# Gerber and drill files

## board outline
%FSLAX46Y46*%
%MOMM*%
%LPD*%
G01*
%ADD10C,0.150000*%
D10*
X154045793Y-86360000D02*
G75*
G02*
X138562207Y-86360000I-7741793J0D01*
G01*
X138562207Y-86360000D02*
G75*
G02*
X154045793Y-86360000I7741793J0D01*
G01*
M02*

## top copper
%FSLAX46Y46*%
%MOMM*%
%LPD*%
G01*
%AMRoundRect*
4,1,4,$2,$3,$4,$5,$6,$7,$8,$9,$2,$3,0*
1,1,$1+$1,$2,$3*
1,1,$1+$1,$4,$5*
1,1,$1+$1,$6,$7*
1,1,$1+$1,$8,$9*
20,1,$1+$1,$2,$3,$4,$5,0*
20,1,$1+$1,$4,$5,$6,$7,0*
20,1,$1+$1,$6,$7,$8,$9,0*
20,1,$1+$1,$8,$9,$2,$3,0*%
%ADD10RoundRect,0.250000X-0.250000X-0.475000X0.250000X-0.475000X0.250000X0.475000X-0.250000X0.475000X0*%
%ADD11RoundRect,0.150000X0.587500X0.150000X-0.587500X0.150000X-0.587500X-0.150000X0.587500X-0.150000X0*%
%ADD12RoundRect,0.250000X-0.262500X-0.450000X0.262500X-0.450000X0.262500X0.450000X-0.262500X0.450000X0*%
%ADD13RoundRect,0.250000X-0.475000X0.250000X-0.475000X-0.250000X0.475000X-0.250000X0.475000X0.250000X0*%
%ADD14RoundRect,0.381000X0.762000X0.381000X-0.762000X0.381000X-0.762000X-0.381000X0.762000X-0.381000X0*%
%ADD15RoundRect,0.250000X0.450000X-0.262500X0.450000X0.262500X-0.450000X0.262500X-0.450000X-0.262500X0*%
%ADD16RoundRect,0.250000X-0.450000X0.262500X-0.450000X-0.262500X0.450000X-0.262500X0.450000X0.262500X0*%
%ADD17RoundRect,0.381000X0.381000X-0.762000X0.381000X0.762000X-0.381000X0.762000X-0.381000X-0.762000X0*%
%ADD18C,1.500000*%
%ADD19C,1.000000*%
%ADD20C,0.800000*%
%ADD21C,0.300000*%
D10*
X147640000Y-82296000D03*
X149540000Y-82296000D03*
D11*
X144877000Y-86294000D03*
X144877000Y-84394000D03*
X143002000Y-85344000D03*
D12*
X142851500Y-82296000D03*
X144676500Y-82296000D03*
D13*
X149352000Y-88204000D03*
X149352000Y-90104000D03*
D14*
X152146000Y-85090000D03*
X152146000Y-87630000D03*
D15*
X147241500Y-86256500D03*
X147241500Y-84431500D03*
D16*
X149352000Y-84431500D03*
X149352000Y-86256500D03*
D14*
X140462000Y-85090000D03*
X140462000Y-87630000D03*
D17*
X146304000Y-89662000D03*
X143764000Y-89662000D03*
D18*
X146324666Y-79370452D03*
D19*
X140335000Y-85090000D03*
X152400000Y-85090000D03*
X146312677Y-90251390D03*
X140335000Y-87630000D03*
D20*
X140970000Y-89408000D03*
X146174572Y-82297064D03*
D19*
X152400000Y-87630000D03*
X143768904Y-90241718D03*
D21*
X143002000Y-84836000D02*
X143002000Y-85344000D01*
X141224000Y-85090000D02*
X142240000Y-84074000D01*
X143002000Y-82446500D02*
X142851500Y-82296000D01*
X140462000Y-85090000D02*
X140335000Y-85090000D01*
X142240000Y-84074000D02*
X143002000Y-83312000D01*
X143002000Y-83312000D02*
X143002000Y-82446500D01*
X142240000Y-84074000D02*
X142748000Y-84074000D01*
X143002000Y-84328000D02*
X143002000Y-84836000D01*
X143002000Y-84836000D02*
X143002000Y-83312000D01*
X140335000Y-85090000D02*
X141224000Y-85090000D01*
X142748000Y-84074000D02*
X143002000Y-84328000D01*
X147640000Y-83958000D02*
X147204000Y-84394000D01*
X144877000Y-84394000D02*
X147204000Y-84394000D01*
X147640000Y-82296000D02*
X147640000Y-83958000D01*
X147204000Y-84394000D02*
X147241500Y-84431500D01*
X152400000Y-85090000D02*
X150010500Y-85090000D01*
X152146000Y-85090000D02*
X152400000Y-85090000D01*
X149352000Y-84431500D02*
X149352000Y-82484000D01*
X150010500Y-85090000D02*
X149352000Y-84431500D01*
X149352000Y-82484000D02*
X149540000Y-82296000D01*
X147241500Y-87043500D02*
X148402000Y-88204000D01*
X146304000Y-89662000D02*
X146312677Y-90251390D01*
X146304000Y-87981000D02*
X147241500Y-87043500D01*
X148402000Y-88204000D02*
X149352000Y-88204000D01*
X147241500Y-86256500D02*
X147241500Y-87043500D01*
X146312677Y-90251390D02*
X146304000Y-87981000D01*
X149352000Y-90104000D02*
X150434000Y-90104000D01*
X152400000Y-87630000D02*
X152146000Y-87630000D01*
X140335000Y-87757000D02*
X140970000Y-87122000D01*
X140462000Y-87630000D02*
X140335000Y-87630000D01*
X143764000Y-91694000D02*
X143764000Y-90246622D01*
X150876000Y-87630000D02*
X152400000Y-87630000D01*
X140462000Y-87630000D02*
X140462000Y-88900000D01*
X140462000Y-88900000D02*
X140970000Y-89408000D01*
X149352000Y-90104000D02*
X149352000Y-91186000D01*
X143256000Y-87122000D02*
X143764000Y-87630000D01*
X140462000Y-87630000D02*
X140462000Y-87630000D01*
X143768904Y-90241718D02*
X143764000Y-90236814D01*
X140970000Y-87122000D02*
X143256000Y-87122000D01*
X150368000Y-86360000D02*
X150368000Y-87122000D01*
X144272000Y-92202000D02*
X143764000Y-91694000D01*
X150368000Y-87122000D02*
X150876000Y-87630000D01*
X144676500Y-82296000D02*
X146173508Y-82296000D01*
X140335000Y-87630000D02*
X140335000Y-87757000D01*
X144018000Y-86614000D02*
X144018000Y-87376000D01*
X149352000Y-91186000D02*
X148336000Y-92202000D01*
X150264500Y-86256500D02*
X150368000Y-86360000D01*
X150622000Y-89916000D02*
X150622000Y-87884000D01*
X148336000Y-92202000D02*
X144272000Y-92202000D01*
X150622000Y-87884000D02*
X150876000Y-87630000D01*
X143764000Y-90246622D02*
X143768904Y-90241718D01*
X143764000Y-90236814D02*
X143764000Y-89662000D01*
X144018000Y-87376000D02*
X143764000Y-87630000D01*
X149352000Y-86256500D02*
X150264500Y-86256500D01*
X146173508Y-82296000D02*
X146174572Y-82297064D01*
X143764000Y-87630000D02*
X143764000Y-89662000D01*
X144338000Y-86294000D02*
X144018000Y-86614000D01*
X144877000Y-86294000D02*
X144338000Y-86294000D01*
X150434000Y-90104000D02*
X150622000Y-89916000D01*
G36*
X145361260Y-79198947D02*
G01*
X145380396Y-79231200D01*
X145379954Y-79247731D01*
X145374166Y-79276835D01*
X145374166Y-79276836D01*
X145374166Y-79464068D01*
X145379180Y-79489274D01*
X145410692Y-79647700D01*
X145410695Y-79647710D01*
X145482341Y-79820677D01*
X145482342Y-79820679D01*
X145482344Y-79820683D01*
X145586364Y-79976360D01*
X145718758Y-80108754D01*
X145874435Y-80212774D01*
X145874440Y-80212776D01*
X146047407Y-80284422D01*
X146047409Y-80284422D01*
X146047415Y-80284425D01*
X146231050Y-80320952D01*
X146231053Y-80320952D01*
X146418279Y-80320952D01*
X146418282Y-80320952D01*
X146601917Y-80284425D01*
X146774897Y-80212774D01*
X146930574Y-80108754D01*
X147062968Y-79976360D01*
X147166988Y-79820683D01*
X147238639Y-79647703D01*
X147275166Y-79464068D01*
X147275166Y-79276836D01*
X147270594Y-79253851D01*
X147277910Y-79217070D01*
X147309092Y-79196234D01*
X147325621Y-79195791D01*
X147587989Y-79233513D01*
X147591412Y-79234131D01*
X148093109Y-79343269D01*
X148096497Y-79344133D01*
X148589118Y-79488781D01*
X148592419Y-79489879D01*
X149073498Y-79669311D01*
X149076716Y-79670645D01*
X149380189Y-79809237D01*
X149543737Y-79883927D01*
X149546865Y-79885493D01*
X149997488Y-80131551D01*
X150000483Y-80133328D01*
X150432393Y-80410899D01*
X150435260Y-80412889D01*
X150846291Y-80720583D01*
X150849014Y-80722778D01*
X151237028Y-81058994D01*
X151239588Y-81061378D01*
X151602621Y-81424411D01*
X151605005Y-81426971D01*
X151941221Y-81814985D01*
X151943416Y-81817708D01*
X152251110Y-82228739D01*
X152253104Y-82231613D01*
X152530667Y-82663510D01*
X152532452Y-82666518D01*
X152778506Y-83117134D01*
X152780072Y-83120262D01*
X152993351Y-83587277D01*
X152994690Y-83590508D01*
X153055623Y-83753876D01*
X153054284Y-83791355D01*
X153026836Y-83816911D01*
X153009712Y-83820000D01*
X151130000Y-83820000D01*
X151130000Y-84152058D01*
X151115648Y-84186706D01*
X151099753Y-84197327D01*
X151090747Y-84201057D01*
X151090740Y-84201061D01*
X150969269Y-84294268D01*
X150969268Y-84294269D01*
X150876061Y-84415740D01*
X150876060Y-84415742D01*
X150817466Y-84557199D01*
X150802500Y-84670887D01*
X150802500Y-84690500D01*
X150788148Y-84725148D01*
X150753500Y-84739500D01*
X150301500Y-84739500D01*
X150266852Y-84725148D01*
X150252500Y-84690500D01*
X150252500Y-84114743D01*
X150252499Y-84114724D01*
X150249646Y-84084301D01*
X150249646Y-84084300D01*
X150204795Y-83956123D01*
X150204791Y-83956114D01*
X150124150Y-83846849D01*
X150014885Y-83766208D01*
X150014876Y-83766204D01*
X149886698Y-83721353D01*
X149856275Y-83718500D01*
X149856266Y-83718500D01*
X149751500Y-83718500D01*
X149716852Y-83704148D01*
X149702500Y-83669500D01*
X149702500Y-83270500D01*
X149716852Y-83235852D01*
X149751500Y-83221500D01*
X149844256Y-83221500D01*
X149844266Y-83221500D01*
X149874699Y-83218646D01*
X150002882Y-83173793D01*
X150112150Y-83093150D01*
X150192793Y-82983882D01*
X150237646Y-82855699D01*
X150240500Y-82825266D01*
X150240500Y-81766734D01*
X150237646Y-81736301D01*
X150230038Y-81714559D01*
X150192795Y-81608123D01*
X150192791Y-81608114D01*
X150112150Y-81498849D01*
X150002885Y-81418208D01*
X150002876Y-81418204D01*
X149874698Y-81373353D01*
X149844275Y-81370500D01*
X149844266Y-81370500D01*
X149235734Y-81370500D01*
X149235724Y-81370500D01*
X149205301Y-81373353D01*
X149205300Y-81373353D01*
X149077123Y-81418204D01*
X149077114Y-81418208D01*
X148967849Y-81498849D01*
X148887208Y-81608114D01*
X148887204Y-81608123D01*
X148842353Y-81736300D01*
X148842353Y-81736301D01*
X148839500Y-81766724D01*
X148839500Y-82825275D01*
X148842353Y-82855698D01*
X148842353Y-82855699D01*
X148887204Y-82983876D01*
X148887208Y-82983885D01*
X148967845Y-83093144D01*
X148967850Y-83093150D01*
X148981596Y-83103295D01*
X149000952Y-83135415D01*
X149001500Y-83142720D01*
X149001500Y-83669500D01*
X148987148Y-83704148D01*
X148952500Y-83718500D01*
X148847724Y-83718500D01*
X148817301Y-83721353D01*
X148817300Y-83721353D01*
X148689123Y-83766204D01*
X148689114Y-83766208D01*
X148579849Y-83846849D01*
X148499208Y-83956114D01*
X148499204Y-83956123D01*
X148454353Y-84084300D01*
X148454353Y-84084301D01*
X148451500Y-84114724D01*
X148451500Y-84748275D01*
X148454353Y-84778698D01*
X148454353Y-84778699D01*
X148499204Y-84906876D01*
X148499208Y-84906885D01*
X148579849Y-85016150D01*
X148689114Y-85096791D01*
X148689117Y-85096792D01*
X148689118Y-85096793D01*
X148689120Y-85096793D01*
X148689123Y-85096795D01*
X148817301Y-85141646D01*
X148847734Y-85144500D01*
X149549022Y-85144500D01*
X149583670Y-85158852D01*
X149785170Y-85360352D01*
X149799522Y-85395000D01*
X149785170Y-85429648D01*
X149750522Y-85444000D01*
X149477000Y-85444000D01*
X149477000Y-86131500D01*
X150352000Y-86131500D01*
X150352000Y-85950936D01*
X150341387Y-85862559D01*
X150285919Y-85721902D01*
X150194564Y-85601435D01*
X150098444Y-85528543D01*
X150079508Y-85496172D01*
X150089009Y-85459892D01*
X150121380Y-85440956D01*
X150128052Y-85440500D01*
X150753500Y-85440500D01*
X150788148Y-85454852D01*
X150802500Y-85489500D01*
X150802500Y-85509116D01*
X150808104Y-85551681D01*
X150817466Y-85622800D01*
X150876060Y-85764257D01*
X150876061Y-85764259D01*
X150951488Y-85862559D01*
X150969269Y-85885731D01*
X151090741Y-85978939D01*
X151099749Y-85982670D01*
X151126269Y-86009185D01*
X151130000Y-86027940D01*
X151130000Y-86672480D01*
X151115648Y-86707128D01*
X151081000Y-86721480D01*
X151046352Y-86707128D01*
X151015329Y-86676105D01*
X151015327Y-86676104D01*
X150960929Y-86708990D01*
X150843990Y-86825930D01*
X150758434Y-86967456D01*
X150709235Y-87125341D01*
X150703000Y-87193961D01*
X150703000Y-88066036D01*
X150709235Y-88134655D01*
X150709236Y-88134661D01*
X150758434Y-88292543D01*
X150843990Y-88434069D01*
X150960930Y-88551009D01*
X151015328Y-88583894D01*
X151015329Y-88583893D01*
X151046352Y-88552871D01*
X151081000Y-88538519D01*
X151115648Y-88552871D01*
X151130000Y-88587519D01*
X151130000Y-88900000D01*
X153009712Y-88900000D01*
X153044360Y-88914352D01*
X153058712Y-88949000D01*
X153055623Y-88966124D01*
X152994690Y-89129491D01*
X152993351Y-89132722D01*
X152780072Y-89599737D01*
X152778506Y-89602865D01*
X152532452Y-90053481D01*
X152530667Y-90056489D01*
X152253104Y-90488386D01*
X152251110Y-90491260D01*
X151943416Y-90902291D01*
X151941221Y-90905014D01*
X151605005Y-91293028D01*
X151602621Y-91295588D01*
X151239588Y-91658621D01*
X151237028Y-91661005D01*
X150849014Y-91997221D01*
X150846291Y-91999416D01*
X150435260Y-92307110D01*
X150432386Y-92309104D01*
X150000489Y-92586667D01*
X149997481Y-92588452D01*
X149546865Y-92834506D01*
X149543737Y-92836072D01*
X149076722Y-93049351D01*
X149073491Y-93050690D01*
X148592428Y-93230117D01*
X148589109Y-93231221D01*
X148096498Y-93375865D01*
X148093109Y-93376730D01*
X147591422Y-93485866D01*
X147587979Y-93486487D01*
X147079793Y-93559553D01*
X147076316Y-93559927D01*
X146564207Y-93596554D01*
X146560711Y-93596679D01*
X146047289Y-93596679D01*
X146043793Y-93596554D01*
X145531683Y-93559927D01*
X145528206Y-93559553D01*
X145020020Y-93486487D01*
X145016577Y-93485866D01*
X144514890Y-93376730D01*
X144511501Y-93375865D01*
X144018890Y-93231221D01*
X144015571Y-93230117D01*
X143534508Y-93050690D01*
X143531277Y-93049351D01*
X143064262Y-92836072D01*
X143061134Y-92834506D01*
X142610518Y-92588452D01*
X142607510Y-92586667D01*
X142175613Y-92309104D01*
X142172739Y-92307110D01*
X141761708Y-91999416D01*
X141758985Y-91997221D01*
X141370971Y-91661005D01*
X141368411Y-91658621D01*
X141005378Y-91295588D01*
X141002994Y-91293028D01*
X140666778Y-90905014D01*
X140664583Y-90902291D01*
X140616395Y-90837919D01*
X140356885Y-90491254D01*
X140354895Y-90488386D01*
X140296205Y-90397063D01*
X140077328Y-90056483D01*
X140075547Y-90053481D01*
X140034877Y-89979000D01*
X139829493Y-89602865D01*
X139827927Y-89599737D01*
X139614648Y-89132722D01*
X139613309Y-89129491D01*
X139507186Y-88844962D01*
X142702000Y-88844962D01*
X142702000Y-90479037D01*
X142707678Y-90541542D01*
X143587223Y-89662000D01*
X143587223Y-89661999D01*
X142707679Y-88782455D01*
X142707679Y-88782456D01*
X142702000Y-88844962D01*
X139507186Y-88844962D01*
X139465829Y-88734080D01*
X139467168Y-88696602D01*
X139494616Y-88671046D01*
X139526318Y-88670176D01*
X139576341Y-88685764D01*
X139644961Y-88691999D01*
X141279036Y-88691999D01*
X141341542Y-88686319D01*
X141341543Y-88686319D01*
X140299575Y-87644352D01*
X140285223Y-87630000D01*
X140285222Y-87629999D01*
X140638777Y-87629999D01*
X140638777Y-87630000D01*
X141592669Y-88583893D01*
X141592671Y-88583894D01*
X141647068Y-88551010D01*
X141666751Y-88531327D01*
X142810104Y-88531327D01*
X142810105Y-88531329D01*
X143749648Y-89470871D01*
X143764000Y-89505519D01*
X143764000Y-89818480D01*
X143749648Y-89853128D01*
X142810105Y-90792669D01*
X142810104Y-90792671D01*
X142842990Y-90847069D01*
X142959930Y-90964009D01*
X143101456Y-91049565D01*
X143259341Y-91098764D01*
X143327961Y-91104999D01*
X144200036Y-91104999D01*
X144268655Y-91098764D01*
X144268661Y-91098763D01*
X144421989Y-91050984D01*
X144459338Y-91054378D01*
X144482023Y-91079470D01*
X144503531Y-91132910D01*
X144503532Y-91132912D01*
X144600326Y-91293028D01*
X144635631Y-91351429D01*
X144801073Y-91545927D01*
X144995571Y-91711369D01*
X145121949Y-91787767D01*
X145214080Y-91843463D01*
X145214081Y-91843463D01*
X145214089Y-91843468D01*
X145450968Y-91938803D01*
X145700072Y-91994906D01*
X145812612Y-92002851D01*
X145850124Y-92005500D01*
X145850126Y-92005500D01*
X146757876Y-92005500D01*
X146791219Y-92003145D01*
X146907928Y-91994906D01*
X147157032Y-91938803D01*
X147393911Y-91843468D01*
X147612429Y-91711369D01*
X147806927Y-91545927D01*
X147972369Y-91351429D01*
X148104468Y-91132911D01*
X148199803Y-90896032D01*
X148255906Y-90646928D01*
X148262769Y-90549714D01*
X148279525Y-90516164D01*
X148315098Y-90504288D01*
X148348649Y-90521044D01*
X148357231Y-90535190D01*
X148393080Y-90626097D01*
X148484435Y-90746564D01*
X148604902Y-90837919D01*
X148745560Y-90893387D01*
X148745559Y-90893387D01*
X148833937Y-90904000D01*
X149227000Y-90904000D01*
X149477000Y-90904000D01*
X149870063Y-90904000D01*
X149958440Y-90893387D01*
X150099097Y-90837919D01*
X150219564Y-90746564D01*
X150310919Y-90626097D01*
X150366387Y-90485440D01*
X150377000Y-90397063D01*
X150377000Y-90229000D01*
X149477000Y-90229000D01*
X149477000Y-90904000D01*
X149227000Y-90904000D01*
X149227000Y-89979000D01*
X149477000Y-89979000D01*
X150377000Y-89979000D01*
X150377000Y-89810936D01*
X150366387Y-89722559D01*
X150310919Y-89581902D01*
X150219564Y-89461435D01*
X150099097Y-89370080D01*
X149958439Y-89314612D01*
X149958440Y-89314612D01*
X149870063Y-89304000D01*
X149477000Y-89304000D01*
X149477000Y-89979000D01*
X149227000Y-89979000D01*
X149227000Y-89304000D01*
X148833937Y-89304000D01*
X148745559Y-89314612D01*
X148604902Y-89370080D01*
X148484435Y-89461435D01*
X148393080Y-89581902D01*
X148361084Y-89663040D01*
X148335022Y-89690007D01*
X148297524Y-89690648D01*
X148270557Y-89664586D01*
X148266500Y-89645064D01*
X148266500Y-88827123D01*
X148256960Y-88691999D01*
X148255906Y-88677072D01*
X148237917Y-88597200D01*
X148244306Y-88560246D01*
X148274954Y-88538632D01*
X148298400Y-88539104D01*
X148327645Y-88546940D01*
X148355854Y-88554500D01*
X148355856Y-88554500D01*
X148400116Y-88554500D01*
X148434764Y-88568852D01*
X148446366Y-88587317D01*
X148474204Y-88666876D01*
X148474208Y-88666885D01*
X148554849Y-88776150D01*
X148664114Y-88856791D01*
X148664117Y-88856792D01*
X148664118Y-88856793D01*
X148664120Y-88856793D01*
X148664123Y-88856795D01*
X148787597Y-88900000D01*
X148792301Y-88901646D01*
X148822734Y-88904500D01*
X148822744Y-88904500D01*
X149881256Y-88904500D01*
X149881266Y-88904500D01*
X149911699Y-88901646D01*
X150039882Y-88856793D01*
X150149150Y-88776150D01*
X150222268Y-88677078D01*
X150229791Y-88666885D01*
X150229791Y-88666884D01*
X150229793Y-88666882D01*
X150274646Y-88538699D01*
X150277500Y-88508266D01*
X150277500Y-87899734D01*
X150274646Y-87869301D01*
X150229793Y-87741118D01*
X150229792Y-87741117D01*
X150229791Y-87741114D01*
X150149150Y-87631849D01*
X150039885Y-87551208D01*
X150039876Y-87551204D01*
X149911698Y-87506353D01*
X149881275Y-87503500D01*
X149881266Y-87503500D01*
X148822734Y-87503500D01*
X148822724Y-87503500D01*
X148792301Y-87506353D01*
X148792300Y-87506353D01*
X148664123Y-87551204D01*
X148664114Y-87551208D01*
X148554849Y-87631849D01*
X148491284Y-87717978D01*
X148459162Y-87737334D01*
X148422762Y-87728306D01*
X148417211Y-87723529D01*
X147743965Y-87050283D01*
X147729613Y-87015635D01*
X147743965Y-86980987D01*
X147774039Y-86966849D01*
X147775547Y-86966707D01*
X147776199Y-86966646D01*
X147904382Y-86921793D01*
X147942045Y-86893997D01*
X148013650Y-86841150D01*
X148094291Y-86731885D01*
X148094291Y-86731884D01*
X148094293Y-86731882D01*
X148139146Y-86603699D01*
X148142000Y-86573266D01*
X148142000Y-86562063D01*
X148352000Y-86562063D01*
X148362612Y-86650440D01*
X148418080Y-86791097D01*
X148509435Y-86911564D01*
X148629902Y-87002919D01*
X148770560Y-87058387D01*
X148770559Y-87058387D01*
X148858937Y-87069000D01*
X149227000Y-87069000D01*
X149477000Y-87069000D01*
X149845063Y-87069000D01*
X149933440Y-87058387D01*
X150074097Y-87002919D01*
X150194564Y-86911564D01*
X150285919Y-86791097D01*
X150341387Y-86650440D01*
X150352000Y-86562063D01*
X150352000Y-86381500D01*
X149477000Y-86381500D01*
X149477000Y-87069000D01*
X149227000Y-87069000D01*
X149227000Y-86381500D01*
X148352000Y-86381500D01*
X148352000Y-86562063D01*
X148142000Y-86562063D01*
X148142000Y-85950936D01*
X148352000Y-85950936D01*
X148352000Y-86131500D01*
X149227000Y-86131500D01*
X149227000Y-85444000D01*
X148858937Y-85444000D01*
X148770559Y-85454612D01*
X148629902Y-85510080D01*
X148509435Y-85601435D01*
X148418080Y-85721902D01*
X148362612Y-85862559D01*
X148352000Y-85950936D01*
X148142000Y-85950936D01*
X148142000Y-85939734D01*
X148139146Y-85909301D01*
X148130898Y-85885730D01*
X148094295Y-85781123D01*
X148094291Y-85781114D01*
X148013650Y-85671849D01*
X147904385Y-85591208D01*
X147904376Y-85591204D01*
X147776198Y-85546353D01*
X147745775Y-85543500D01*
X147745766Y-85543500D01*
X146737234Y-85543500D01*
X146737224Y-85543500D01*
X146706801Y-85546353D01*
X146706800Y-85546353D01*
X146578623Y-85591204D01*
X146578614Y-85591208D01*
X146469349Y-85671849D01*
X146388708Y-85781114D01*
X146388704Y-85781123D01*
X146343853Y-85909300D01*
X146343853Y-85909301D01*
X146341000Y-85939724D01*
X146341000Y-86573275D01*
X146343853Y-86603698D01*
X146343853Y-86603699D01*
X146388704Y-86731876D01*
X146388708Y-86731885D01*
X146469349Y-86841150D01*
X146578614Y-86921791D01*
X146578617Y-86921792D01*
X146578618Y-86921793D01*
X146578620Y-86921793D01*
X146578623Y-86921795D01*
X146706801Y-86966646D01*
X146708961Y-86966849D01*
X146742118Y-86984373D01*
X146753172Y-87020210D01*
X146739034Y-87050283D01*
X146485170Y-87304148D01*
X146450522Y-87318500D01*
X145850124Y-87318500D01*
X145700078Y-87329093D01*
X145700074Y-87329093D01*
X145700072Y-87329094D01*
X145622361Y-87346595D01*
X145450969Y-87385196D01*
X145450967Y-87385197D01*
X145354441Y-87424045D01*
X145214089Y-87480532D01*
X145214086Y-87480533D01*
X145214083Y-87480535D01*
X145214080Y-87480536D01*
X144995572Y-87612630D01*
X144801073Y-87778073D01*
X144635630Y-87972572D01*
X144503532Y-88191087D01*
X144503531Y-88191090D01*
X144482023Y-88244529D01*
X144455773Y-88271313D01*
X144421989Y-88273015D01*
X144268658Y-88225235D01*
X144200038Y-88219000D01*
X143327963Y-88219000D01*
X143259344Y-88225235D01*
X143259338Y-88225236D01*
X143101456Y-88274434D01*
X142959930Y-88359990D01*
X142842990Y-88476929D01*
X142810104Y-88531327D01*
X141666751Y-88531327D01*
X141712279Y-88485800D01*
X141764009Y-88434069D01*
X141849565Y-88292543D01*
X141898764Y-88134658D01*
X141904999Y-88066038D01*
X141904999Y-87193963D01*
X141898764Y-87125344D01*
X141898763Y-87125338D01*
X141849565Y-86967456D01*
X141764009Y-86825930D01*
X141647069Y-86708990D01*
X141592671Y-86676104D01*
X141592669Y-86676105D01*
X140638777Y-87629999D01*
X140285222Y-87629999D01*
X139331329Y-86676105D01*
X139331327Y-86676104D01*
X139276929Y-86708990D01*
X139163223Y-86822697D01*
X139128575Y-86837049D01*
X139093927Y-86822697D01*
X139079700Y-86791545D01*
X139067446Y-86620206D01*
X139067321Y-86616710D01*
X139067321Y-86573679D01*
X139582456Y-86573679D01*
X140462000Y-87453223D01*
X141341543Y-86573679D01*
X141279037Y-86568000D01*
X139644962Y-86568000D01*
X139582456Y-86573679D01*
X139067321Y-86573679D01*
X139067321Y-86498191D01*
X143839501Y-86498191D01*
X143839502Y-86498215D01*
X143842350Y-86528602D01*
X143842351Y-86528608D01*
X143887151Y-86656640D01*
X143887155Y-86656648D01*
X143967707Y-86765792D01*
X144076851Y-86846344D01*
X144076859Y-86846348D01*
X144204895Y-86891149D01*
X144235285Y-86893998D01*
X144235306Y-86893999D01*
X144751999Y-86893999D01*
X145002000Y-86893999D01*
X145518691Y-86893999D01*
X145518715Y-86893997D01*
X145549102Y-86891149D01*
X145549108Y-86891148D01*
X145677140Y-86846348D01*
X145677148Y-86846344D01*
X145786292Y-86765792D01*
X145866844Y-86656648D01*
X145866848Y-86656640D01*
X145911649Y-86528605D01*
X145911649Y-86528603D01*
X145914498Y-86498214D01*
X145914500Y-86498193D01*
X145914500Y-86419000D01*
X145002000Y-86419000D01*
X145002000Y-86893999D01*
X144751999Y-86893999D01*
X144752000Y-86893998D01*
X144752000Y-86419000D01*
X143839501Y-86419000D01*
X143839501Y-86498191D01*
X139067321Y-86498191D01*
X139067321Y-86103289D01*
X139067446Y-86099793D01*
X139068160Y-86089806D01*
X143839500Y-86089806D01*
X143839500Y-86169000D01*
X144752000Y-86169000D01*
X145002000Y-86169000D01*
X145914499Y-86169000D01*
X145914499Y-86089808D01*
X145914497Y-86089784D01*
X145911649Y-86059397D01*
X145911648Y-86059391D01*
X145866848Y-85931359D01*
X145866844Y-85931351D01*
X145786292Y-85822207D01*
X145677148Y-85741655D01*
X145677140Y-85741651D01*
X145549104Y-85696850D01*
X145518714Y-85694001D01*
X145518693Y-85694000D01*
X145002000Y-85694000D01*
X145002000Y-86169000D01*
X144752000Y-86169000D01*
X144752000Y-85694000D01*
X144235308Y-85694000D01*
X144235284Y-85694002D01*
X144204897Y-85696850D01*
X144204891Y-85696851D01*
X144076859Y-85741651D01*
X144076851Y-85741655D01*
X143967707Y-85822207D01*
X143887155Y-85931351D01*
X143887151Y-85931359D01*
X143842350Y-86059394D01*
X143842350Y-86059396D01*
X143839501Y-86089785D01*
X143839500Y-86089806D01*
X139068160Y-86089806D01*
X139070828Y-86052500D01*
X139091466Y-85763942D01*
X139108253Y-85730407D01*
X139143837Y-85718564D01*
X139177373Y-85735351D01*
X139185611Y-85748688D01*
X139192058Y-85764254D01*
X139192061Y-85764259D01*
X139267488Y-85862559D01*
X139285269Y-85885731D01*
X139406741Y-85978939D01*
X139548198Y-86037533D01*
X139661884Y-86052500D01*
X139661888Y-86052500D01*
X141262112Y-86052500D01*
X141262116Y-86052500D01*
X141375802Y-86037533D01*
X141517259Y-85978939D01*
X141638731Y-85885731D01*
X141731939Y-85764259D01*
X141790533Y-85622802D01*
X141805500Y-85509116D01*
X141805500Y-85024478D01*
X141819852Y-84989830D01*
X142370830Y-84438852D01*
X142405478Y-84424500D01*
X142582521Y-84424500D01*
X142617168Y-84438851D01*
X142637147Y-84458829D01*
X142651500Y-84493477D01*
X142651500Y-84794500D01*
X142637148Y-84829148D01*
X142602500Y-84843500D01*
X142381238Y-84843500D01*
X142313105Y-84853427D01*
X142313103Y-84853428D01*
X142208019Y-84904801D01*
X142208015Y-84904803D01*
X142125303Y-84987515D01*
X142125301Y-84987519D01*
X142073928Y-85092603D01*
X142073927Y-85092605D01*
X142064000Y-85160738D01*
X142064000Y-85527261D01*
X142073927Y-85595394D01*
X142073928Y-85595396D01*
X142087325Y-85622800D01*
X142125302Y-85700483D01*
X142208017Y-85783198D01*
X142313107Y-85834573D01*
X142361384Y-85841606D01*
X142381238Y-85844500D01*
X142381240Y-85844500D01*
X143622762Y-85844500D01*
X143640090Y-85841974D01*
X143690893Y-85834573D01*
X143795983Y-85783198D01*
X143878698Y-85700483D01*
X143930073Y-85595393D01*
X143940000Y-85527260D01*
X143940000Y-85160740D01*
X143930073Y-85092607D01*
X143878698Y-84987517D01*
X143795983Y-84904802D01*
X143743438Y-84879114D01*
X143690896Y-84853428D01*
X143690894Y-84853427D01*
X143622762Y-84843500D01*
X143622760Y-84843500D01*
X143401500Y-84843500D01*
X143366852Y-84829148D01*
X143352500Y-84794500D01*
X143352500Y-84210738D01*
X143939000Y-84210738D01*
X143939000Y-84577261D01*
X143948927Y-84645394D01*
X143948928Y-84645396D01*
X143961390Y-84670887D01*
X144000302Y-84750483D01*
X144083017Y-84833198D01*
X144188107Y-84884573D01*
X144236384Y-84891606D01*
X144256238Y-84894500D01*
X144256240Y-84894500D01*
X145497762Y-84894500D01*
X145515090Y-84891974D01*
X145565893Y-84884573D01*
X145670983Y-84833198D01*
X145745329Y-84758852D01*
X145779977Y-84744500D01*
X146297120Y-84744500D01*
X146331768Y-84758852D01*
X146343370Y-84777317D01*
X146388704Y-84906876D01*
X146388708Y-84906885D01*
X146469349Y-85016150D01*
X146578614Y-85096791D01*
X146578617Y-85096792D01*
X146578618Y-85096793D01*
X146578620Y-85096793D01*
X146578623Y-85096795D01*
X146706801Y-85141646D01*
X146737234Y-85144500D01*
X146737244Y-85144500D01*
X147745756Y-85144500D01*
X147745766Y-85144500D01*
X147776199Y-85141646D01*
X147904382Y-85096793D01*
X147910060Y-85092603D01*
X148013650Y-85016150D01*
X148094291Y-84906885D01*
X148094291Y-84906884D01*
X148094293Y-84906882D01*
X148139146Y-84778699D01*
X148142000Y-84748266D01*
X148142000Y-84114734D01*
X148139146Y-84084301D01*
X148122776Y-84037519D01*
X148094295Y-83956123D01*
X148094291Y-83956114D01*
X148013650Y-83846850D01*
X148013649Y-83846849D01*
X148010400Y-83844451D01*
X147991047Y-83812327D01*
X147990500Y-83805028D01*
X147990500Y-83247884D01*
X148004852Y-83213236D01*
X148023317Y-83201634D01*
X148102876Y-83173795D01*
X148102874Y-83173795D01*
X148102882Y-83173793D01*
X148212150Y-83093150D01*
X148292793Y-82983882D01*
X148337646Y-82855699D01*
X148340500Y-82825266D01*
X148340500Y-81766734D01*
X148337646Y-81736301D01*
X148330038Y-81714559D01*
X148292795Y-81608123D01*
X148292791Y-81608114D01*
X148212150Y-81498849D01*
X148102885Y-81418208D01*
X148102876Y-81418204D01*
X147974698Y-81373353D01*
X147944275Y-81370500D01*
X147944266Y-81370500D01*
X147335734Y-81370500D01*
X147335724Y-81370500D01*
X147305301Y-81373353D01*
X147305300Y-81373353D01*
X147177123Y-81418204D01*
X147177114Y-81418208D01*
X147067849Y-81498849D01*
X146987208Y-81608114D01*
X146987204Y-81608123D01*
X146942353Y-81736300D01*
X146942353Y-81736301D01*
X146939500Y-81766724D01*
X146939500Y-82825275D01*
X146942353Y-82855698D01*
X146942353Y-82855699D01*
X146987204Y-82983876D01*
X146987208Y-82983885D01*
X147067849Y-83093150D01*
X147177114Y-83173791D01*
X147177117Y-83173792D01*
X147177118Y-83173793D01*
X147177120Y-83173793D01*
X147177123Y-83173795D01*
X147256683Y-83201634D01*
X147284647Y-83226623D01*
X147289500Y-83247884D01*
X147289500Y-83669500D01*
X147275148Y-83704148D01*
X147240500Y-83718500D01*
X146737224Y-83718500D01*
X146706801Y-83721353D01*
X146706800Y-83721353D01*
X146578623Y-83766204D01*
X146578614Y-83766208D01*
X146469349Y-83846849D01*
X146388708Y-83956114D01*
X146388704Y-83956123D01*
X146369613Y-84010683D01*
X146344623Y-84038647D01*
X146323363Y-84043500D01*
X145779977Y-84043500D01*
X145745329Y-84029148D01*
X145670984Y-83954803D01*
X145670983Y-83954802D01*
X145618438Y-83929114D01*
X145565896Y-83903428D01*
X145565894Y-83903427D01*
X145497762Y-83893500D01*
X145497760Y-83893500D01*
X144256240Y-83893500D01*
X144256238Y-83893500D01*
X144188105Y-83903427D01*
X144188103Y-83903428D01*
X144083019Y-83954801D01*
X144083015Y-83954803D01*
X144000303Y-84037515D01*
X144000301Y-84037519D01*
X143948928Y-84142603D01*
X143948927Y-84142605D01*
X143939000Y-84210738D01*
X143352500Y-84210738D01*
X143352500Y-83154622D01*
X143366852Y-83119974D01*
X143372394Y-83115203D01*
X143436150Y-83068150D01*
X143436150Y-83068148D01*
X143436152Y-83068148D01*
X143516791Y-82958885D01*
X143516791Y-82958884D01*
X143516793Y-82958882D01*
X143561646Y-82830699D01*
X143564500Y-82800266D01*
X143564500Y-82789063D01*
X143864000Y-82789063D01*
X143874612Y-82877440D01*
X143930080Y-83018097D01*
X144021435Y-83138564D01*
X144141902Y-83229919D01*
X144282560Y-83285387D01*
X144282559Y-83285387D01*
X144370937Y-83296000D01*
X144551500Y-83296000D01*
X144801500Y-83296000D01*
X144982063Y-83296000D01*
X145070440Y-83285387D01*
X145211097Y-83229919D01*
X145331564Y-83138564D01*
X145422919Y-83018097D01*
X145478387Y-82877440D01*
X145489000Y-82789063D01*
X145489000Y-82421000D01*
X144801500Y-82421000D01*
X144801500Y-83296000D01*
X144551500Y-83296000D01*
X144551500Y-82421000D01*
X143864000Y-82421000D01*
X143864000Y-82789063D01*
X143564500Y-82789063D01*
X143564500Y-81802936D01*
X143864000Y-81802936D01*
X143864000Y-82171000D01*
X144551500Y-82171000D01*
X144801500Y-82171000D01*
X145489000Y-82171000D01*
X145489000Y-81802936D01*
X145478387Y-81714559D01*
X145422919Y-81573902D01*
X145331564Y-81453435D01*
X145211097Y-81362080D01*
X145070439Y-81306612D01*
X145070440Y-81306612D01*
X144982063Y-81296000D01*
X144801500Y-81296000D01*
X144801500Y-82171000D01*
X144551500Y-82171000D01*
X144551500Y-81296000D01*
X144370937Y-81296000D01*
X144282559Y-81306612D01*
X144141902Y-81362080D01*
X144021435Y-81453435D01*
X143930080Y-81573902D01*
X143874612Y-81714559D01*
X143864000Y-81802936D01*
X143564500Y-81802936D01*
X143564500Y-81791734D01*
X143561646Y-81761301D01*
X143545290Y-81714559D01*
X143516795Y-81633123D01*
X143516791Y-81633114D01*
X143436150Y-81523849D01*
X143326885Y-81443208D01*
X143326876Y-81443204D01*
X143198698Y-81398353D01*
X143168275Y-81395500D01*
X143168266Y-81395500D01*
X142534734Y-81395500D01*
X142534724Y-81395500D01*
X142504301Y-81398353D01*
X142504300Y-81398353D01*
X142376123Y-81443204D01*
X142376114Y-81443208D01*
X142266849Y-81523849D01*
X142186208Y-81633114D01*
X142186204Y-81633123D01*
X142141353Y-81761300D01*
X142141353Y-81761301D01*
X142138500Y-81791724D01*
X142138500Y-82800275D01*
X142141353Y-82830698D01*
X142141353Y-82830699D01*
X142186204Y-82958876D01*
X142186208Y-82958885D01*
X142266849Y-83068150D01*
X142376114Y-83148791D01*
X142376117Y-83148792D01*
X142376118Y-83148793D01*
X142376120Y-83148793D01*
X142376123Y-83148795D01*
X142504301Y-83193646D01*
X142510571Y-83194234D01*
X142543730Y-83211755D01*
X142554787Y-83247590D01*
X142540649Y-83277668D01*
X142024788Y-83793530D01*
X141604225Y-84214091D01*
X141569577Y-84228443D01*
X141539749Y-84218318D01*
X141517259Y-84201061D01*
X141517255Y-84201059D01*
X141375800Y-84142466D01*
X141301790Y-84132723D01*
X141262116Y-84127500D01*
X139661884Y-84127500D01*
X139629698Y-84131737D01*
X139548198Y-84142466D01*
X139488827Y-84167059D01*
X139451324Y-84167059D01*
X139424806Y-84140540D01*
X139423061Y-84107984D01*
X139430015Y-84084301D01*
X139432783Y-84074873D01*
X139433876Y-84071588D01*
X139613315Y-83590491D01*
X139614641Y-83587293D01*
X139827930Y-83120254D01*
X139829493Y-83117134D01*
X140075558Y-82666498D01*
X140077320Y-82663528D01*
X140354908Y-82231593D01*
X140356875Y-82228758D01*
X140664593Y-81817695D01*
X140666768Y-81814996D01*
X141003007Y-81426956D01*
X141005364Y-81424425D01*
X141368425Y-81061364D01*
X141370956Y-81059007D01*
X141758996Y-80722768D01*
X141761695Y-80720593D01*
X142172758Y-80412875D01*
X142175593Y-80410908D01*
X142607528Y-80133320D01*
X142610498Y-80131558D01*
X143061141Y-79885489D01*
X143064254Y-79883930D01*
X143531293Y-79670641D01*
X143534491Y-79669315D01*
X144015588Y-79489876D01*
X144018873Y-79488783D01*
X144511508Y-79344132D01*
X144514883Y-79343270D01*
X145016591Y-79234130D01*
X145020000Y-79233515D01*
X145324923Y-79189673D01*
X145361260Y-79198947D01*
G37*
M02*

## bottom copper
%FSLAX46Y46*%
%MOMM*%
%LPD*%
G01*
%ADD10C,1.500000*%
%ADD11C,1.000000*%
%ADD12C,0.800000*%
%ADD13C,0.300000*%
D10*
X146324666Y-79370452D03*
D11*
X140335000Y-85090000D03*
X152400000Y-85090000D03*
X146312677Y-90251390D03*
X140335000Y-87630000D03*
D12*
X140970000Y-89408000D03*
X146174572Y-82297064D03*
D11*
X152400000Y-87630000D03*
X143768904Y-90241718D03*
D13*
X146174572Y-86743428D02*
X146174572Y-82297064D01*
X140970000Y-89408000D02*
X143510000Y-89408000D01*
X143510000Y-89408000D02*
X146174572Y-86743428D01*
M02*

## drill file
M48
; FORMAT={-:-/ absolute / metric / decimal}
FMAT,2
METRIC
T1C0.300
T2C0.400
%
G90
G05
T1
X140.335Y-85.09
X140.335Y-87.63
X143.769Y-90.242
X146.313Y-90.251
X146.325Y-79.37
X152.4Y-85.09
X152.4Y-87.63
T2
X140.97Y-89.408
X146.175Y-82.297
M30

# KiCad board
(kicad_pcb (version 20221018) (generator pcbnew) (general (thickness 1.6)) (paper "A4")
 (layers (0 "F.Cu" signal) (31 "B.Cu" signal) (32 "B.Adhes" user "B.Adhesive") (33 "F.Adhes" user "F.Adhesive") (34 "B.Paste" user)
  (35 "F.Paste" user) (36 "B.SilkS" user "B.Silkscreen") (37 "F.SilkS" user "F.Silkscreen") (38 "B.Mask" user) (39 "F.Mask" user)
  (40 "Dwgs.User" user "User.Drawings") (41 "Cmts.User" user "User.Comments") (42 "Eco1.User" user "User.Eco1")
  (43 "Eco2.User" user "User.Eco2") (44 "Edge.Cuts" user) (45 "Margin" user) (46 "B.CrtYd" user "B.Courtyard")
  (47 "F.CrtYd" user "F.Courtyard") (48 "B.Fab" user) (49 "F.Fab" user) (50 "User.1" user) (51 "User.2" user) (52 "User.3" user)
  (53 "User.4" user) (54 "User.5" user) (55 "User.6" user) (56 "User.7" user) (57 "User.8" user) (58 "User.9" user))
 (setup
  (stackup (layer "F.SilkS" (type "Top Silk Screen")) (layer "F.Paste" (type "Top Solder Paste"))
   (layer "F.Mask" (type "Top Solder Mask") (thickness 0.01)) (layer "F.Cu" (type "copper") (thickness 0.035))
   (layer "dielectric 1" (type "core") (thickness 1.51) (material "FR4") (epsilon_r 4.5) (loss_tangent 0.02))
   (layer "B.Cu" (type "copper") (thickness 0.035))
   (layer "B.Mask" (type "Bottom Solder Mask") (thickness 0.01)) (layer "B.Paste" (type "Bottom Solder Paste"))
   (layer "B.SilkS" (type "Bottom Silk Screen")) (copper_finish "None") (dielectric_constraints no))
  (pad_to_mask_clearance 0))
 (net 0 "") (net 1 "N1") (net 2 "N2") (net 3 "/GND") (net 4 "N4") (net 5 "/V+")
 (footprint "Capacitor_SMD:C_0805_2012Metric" (layer "F.Cu") (at 148.59 82.296)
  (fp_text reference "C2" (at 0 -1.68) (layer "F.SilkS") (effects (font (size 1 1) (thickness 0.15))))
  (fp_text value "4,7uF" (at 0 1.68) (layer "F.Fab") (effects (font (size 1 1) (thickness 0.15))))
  (pad "1" smd roundrect (at -0.95 0) (size 1 1.45) (layers "F.Cu" "F.Paste" "F.Mask") (roundrect_rratio 0.25) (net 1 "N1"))
  (pad "2" smd roundrect (at 0.95 0) (size 1 1.45) (layers "F.Cu" "F.Paste" "F.Mask") (roundrect_rratio 0.25) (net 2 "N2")))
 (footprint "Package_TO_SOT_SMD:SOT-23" (layer "F.Cu") (at 143.9395 85.344 180)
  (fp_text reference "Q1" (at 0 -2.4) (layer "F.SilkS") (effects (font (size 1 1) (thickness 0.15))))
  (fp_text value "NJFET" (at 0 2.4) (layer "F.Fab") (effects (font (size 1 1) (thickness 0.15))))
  (pad "1" smd roundrect (at -0.9375 -0.95 180) (size 1.475 0.6) (layers "F.Cu" "F.Paste" "F.Mask") (roundrect_rratio 0.25) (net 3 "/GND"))
  (pad "2" smd roundrect (at -0.9375 0.95 180) (size 1.475 0.6) (layers "F.Cu" "F.Paste" "F.Mask") (roundrect_rratio 0.25) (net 1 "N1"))
  (pad "3" smd roundrect (at 0.9375 0 180) (size 1.475 0.6) (layers "F.Cu" "F.Paste" "F.Mask") (roundrect_rratio 0.25) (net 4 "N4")))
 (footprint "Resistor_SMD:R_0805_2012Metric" (layer "F.Cu") (at 143.764 82.296)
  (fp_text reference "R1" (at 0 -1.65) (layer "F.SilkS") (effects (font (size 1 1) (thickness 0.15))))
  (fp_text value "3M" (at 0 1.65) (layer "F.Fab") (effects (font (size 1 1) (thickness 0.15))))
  (pad "1" smd roundrect (at -0.9125 0) (size 1.025 1.4) (layers "F.Cu" "F.Paste" "F.Mask") (roundrect_rratio 0.243902) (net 4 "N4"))
  (pad "2" smd roundrect (at 0.9125 0) (size 1.025 1.4) (layers "F.Cu" "F.Paste" "F.Mask") (roundrect_rratio 0.243902) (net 3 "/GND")))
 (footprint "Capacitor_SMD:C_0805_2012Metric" (layer "F.Cu") (at 149.352 89.154 -90)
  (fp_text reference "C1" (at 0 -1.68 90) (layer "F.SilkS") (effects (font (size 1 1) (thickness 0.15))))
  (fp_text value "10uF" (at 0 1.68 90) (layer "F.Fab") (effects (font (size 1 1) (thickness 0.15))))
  (pad "1" smd roundrect (at -0.95 0 270) (size 1 1.45) (layers "F.Cu" "F.Paste" "F.Mask") (roundrect_rratio 0.25) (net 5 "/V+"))
  (pad "2" smd roundrect (at 0.95 0 270) (size 1 1.45) (layers "F.Cu" "F.Paste" "F.Mask") (roundrect_rratio 0.25) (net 3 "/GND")))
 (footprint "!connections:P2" (layer "F.Cu") (at 152.146 85.09 180)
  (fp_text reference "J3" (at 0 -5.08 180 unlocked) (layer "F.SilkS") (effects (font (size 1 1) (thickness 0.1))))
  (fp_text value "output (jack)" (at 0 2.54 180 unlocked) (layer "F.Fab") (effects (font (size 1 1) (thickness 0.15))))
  (pad "1" smd roundrect (at 0 0 180) (size 2.286 1.524) (layers "F.Cu" "F.Paste" "F.Mask") (roundrect_rratio 0.25) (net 2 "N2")
   (thermal_bridge_angle 45))
  (pad "2" smd roundrect (at 0 -2.54 180) (size 2.286 1.524) (layers "F.Cu" "F.Paste" "F.Mask") (roundrect_rratio 0.25) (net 3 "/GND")
   (thermal_bridge_angle 45)))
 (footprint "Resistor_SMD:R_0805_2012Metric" (layer "F.Cu") (at 147.2415 85.344 90)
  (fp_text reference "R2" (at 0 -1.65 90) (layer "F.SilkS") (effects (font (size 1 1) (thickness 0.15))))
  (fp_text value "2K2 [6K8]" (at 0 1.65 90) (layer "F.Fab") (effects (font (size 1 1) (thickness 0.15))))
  (pad "1" smd roundrect (at -0.9125 0 90) (size 1.025 1.4) (layers "F.Cu" "F.Paste" "F.Mask") (roundrect_rratio 0.243902) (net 5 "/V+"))
  (pad "2" smd roundrect (at 0.9125 0 90) (size 1.025 1.4) (layers "F.Cu" "F.Paste" "F.Mask") (roundrect_rratio 0.243902) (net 1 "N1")))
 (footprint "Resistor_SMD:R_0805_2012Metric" (layer "F.Cu") (at 149.352 85.344 -90)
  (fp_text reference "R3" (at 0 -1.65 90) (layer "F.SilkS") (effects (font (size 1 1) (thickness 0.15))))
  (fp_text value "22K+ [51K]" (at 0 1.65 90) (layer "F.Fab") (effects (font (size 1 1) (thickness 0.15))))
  (pad "1" smd roundrect (at -0.9125 0 270) (size 1.025 1.4) (layers "F.Cu" "F.Paste" "F.Mask") (roundrect_rratio 0.243902) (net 2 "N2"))
  (pad "2" smd roundrect (at 0.9125 0 270) (size 1.025 1.4) (layers "F.Cu" "F.Paste" "F.Mask") (roundrect_rratio 0.243902) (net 3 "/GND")))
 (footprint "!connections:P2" (layer "F.Cu") (at 140.462 85.09 180)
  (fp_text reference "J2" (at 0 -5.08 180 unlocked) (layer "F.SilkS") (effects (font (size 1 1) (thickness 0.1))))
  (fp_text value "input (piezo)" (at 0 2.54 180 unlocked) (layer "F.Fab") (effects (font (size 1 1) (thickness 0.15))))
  (pad "1" smd roundrect (at 0 0 180) (size 2.286 1.524) (layers "F.Cu" "F.Paste" "F.Mask") (roundrect_rratio 0.25) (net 4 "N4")
   (thermal_bridge_angle 45))
  (pad "2" smd roundrect (at 0 -2.54 180) (size 2.286 1.524) (layers "F.Cu" "F.Paste" "F.Mask") (roundrect_rratio 0.25) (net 3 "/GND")
   (thermal_bridge_angle 45)))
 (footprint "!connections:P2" (layer "F.Cu") (at 146.304 89.662 90) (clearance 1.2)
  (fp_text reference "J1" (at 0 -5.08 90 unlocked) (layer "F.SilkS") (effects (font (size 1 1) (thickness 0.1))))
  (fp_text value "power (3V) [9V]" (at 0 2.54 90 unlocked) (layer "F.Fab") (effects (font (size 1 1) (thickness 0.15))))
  (pad "1" smd roundrect (at 0 0 90) (size 2.286 1.524) (layers "F.Cu" "F.Paste" "F.Mask") (roundrect_rratio 0.25) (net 5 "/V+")
   (thermal_bridge_angle 45))
  (pad "2" smd roundrect (at 0 -2.54 90) (size 2.286 1.524) (layers "F.Cu" "F.Paste" "F.Mask") (roundrect_rratio 0.25) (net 3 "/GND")
   (thermal_bridge_angle 45)))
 (gr_circle (center 146.304 86.36) (end 151.384 80.518) (stroke (width 0.15) (type default)) (fill none) (layer "Edge.Cuts"))
 (via (at 146.324666 79.370452) (size 1.5) (drill 0.3) (layers "F.Cu" "B.Cu") (free) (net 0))
 (segment (start 143.002 84.836) (end 143.002 85.344) (width 0.3) (layer "F.Cu") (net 4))
 (segment (start 141.224 85.09) (end 142.24 84.074) (width 0.3) (layer "F.Cu") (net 4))
 (segment (start 143.002 82.4465) (end 142.8515 82.296) (width 0.3) (layer "F.Cu") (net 4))
 (segment (start 140.462 85.09) (end 140.335 85.09) (width 0.3) (layer "F.Cu") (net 4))
 (segment (start 142.24 84.074) (end 143.002 83.312) (width 0.3) (layer "F.Cu") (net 4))
 (segment (start 143.002 83.312) (end 143.002 82.4465) (width 0.3) (layer "F.Cu") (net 4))
 (segment (start 142.24 84.074) (end 142.748 84.074) (width 0.3) (layer "F.Cu") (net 4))
 (segment (start 143.002 84.328) (end 143.002 84.836) (width 0.3) (layer "F.Cu") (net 4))
 (segment (start 143.002 84.836) (end 143.002 83.312) (width 0.3) (layer "F.Cu") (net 4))
 (segment (start 140.335 85.09) (end 141.224 85.09) (width 0.3) (layer "F.Cu") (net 4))
 (segment (start 142.748 84.074) (end 143.002 84.328) (width 0.3) (layer "F.Cu") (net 4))
 (via (at 140.335 85.09) (size 1) (drill 0.3) (layers "F.Cu" "B.Cu") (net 4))
 (segment (start 147.64 83.958) (end 147.204 84.394) (width 0.3) (layer "F.Cu") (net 1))
 (segment (start 144.877 84.394) (end 147.204 84.394) (width 0.3) (layer "F.Cu") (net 1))
 (segment (start 147.64 82.296) (end 147.64 83.958) (width 0.3) (layer "F.Cu") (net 1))
 (segment (start 147.204 84.394) (end 147.2415 84.4315) (width 0.3) (layer "F.Cu") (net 1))
 (segment (start 152.4 85.09) (end 150.0105 85.09) (width 0.3) (layer "F.Cu") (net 2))
 (segment (start 152.146 85.09) (end 152.4 85.09) (width 0.3) (layer "F.Cu") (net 2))
 (segment (start 149.352 84.4315) (end 149.352 82.484) (width 0.3) (layer "F.Cu") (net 2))
 (segment (start 150.0105 85.09) (end 149.352 84.4315) (width 0.3) (layer "F.Cu") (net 2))
 (segment (start 149.352 82.484) (end 149.54 82.296) (width 0.3) (layer "F.Cu") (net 2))
 (via (at 152.4 85.09) (size 1) (drill 0.3) (layers "F.Cu" "B.Cu") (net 2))
 (segment (start 147.2415 87.0435) (end 148.402 88.204) (width 0.3) (layer "F.Cu") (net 5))
 (segment (start 146.304 89.662) (end 146.312677 90.25139) (width 0.3) (layer "F.Cu") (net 5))
 (segment (start 146.304 87.981) (end 147.2415 87.0435) (width 0.3) (layer "F.Cu") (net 5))
 (segment (start 148.402 88.204) (end 149.352 88.204) (width 0.3) (layer "F.Cu") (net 5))
 (segment (start 147.2415 86.2565) (end 147.2415 87.0435) (width 0.3) (layer "F.Cu") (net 5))
 (segment (start 146.312677 90.25139) (end 146.304 87.981) (width 0.3) (layer "F.Cu") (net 5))
 (via (at 146.312677 90.25139) (size 1) (drill 0.3) (layers "F.Cu" "B.Cu") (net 5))
 (segment (start 149.352 90.104) (end 150.434 90.104) (width 0.3) (layer "F.Cu") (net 3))
 (segment (start 152.4 87.63) (end 152.146 87.63) (width 0.3) (layer "F.Cu") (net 3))
 (segment (start 140.335 87.757) (end 140.97 87.122) (width 0.3) (layer "F.Cu") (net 3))
 (segment (start 140.462 87.63) (end 140.335 87.63) (width 0.3) (layer "F.Cu") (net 3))
 (segment (start 143.764 91.694) (end 143.764 90.246622) (width 0.3) (layer "F.Cu") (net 3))
 (segment (start 150.876 87.63) (end 152.4 87.63) (width 0.3) (layer "F.Cu") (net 3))
 (segment (start 140.462 87.63) (end 140.462 88.9) (width 0.3) (layer "F.Cu") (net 3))
 (segment (start 140.462 88.9) (end 140.97 89.408) (width 0.3) (layer "F.Cu") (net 3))
 (segment (start 149.352 90.104) (end 149.352 91.186) (width 0.3) (layer "F.Cu") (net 3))
 (segment (start 143.256 87.122) (end 143.764 87.63) (width 0.3) (layer "F.Cu") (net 3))
 (segment (start 140.462 87.63) (end 140.462 87.63) (width 0.3) (layer "F.Cu") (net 3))
 (segment (start 143.768904 90.241718) (end 143.764 90.236814) (width 0.3) (layer "F.Cu") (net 3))
 (segment (start 140.97 87.122) (end 143.256 87.122) (width 0.3) (layer "F.Cu") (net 3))
 (segment (start 150.368 86.36) (end 150.368 87.122) (width 0.3) (layer "F.Cu") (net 3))
 (segment (start 144.272 92.202) (end 143.764 91.694) (width 0.3) (layer "F.Cu") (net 3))
 (segment (start 150.368 87.122) (end 150.876 87.63) (width 0.3) (layer "F.Cu") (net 3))
 (segment (start 144.6765 82.296) (end 146.173508 82.296) (width 0.3) (layer "F.Cu") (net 3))
 (segment (start 140.335 87.63) (end 140.335 87.757) (width 0.3) (layer "F.Cu") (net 3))
 (segment (start 144.018 86.614) (end 144.018 87.376) (width 0.3) (layer "F.Cu") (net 3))
 (segment (start 149.352 91.186) (end 148.336 92.202) (width 0.3) (layer "F.Cu") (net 3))
 (segment (start 150.2645 86.2565) (end 150.368 86.36) (width 0.3) (layer "F.Cu") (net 3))
 (segment (start 150.622 89.916) (end 150.622 87.884) (width 0.3) (layer "F.Cu") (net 3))
 (segment (start 148.336 92.202) (end 144.272 92.202) (width 0.3) (layer "F.Cu") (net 3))
 (segment (start 150.622 87.884) (end 150.876 87.63) (width 0.3) (layer "F.Cu") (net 3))
 (segment (start 143.764 90.246622) (end 143.768904 90.241718) (width 0.3) (layer "F.Cu") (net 3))
 (segment (start 143.764 90.236814) (end 143.764 89.662) (width 0.3) (layer "F.Cu") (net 3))
 (segment (start 144.018 87.376) (end 143.764 87.63) (width 0.3) (layer "F.Cu") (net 3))
 (segment (start 149.352 86.2565) (end 150.2645 86.2565) (width 0.3) (layer "F.Cu") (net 3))
 (segment (start 146.173508 82.296) (end 146.174572 82.297064) (width 0.3) (layer "F.Cu") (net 3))
 (segment (start 143.764 87.63) (end 143.764 89.662) (width 0.3) (layer "F.Cu") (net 3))
 (segment (start 144.338 86.294) (end 144.018 86.614) (width 0.3) (layer "F.Cu") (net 3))
 (segment (start 144.877 86.294) (end 144.338 86.294) (width 0.3) (layer "F.Cu") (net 3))
 (segment (start 150.434 90.104) (end 150.622 89.916) (width 0.3) (layer "F.Cu") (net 3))
 (via (at 140.335 87.63) (size 1) (drill 0.3) (layers "F.Cu" "B.Cu") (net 3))
 (via (at 140.97 89.408) (size 0.8) (drill 0.4) (layers "F.Cu" "B.Cu") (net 3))
 (via (at 146.174572 82.297064) (size 0.8) (drill 0.4) (layers "F.Cu" "B.Cu") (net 3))
 (via (at 152.4 87.63) (size 1) (drill 0.3) (layers "F.Cu" "B.Cu") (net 3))
 (via (at 143.768904 90.241718) (size 1) (drill 0.3) (layers "F.Cu" "B.Cu") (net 3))
 (segment (start 146.174572 86.743428) (end 146.174572 82.297064) (width 0.3) (layer "B.Cu") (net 3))
 (segment (start 140.97 89.408) (end 143.51 89.408) (width 0.3) (layer "B.Cu") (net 3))
 (segment (start 143.51 89.408) (end 146.174572 86.743428) (width 0.3) (layer "B.Cu") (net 3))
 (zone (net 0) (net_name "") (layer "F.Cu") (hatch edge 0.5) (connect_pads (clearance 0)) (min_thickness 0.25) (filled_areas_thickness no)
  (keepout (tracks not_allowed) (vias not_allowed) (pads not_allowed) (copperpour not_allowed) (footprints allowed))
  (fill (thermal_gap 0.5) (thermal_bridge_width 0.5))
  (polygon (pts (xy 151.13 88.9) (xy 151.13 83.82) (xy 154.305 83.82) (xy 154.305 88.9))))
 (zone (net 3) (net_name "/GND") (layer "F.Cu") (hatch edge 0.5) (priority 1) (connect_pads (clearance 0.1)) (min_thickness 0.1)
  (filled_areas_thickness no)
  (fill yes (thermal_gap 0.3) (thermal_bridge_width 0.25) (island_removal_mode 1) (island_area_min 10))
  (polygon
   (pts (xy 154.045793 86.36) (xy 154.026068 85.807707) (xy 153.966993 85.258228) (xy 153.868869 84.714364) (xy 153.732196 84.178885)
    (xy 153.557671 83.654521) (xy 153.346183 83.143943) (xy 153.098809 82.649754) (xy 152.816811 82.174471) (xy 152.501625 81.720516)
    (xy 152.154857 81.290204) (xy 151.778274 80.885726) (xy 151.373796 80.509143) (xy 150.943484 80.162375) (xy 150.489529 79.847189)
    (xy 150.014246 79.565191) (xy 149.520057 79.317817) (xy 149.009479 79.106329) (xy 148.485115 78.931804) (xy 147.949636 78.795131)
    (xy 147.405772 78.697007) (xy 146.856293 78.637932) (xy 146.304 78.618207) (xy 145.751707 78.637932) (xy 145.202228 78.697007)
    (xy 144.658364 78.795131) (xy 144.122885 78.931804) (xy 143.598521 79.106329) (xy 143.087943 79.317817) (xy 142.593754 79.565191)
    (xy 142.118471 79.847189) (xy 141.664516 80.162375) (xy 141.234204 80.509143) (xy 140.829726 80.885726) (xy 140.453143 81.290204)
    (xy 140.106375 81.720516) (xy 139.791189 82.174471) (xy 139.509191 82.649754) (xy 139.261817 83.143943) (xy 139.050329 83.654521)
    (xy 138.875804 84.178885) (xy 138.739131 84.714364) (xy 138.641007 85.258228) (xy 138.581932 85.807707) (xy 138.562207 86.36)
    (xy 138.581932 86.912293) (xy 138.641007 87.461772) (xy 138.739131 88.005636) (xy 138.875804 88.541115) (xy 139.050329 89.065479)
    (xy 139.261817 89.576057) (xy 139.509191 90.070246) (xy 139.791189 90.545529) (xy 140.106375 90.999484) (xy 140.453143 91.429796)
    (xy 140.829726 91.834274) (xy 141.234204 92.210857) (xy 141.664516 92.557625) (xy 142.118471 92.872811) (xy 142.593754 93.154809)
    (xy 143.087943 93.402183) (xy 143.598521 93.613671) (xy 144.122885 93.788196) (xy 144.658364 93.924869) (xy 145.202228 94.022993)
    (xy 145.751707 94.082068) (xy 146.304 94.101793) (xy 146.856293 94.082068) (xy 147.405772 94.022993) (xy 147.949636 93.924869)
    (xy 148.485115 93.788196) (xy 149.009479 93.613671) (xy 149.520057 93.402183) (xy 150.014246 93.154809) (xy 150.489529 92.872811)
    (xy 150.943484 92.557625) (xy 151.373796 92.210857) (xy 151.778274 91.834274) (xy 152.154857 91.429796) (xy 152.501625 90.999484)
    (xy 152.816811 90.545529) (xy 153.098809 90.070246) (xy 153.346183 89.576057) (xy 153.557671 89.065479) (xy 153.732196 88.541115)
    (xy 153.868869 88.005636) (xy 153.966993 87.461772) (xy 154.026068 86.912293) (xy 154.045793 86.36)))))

